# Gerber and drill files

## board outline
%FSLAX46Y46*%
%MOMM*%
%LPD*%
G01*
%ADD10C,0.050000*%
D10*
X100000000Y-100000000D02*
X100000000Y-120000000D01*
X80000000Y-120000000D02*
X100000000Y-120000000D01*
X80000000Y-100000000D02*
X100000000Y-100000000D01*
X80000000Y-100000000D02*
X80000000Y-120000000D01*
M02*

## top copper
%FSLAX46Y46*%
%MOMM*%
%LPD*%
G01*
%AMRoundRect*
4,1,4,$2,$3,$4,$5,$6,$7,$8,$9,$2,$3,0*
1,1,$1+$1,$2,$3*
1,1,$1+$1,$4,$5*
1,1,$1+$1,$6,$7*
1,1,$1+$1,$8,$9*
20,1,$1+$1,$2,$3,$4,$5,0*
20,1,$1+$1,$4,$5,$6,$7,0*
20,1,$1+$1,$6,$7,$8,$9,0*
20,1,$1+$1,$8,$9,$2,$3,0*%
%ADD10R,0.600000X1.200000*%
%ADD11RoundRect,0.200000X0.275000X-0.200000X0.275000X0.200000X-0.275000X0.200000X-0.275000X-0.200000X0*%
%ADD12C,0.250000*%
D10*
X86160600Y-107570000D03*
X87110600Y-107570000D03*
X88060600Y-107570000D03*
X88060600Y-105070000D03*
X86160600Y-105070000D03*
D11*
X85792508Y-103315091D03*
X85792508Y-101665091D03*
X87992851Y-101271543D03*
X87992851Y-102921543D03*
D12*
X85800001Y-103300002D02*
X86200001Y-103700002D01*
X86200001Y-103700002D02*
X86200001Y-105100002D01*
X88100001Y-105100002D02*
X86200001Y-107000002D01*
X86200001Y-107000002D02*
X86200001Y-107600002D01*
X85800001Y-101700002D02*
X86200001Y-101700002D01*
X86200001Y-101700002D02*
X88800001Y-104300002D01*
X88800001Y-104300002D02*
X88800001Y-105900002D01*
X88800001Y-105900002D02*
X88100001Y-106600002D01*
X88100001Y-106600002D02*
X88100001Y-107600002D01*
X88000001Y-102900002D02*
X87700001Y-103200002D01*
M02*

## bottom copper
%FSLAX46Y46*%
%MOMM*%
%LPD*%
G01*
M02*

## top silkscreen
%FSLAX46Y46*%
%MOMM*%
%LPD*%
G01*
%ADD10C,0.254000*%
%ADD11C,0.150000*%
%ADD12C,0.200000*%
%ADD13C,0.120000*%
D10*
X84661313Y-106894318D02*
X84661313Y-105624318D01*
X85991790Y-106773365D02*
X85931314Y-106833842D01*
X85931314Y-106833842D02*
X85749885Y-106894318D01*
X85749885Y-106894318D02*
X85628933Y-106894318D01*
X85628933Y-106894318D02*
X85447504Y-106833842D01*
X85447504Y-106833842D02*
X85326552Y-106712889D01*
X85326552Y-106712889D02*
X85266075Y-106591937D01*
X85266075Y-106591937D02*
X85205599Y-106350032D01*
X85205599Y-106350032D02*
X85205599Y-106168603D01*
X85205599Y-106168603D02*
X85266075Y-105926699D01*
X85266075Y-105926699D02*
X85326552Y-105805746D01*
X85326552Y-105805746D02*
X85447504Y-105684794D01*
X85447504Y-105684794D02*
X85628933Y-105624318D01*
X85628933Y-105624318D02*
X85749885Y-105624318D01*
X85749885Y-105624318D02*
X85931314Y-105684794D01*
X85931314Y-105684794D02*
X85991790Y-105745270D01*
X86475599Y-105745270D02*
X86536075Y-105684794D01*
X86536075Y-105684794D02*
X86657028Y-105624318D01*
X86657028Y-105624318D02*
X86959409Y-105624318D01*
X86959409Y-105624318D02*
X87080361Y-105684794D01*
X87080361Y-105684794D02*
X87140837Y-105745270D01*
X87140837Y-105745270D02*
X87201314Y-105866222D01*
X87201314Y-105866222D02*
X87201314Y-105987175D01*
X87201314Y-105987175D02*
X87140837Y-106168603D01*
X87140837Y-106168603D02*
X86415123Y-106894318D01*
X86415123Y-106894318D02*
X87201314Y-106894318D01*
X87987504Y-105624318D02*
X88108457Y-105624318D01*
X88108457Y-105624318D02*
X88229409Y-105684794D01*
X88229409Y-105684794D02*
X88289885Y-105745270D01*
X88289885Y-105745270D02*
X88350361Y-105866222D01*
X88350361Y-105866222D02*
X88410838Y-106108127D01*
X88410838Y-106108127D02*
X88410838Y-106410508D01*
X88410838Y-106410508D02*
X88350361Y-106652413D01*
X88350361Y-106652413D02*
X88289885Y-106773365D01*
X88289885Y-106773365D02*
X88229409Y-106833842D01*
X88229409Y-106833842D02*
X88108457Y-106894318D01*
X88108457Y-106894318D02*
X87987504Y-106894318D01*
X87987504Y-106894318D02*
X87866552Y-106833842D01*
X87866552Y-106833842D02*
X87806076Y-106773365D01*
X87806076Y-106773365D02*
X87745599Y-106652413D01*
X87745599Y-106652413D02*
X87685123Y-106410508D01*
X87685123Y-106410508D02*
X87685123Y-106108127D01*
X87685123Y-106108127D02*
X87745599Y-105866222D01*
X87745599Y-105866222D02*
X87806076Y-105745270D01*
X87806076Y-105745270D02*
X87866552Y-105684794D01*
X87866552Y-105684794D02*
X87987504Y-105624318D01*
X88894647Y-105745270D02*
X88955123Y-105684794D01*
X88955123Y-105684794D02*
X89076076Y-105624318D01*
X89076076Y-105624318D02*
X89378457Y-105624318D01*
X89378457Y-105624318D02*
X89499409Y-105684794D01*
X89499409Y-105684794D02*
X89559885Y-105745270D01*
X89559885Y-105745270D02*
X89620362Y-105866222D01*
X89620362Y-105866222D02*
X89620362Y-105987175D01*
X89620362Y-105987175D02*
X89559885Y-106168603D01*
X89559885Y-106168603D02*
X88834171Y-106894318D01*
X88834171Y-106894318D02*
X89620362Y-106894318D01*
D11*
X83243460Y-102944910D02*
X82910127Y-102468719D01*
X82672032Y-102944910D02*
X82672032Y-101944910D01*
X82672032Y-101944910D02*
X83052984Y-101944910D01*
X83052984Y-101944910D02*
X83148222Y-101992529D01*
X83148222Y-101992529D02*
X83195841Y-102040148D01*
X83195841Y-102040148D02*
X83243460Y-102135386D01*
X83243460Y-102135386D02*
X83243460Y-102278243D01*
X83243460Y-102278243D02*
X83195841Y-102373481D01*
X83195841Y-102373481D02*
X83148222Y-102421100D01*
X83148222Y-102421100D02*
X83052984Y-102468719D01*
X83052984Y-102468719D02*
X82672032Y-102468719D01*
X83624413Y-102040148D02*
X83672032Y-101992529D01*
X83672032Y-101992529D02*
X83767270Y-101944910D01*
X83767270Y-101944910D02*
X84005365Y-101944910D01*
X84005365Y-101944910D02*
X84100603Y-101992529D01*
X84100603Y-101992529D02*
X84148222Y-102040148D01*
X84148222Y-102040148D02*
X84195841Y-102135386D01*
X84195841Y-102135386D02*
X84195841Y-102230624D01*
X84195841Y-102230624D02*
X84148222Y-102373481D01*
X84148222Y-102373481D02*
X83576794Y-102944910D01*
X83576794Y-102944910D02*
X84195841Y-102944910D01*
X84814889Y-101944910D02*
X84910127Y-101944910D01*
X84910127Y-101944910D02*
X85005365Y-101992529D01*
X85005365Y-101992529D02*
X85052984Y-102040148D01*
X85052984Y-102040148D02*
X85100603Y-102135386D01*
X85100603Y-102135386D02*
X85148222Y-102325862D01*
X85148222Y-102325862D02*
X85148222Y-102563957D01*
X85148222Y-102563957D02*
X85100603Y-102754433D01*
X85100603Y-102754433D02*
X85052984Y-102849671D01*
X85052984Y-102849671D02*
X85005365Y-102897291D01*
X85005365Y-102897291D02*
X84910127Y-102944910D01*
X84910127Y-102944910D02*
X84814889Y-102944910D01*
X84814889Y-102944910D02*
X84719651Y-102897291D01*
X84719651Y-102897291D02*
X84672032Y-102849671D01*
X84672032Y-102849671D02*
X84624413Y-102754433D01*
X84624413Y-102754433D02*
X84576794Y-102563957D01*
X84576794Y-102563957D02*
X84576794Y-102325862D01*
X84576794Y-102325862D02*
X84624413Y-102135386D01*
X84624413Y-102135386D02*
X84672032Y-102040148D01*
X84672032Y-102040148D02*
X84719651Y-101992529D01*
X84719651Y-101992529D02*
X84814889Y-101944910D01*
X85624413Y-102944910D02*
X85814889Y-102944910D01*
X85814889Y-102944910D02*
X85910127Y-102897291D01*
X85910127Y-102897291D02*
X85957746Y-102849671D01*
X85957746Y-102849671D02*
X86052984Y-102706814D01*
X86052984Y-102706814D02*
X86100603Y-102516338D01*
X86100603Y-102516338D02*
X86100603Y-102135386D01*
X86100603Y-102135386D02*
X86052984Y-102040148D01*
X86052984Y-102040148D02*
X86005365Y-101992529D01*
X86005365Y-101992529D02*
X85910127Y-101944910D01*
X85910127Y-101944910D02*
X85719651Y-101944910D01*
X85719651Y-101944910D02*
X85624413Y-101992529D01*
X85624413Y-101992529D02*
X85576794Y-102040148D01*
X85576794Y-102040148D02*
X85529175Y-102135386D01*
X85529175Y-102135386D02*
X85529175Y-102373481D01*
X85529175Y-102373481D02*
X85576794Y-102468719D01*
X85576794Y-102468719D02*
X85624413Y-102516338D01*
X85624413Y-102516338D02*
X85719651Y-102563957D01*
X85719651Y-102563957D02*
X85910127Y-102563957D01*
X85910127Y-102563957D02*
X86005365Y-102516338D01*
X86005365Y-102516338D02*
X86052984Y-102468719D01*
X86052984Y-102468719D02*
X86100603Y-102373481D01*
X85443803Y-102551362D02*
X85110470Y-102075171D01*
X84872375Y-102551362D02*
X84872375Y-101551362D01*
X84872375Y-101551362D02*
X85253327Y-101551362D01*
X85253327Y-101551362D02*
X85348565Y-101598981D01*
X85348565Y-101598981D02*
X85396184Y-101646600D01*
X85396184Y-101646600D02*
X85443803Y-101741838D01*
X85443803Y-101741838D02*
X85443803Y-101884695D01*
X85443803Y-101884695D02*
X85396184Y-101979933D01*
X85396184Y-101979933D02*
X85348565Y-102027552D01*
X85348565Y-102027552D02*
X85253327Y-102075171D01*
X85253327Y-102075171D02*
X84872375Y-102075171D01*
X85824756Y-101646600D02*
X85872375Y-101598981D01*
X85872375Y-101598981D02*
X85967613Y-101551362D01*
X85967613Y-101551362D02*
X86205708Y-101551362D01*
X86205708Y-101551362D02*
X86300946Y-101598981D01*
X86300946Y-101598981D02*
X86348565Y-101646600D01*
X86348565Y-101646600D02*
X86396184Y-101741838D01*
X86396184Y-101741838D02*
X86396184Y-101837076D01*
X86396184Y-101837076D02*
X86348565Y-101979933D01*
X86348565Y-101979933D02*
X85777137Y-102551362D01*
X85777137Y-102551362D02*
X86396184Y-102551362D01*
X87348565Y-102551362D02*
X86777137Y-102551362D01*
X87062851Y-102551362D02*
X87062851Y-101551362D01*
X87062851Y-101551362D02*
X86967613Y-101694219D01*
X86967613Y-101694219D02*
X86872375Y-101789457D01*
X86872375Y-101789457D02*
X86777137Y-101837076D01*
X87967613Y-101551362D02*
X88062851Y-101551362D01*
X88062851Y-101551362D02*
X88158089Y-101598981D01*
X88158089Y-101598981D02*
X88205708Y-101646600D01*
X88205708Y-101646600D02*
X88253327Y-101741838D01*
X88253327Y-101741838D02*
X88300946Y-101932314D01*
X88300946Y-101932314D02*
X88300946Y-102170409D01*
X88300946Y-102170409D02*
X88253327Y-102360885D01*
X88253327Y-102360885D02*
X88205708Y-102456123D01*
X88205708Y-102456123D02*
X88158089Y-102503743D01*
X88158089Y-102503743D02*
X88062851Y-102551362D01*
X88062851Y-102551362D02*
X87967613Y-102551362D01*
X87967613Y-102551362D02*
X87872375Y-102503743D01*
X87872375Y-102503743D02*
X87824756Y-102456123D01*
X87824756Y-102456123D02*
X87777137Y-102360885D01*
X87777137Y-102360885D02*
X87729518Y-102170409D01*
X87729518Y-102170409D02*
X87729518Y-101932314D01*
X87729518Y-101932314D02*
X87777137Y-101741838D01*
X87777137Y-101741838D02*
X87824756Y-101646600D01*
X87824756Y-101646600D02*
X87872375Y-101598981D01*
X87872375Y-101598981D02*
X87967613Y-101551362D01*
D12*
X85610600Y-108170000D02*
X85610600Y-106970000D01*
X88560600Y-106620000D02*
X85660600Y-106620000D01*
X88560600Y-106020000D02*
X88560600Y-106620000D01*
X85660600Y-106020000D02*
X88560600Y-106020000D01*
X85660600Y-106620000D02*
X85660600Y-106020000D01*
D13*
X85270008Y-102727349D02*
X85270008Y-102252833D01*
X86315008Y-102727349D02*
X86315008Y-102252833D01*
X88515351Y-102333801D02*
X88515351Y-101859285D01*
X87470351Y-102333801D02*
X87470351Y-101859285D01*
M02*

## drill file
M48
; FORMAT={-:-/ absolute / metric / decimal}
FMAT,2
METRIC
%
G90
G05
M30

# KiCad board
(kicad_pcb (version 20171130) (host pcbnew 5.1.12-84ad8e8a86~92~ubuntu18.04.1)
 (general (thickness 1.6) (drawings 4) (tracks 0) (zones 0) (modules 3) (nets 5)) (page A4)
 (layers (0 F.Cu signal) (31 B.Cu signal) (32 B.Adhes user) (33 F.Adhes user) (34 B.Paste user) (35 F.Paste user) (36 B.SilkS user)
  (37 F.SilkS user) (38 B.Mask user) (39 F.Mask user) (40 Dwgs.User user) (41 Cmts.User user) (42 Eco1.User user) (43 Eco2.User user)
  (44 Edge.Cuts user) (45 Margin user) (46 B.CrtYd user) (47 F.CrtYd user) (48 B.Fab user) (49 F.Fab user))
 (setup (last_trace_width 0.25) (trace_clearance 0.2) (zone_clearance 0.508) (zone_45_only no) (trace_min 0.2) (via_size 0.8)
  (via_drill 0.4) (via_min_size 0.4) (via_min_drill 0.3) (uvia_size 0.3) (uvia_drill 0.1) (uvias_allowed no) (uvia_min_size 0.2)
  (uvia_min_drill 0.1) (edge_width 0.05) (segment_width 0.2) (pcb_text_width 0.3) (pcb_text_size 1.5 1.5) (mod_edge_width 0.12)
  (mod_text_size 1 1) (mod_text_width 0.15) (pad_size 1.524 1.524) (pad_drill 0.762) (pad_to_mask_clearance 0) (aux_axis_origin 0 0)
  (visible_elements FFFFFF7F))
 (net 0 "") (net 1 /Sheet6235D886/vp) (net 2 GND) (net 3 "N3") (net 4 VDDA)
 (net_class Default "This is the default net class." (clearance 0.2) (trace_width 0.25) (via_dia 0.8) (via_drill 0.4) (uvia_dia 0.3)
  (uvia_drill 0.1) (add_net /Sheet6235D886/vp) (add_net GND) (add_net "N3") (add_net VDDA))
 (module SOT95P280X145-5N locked (layer F.Cu) (at 87.110600 106.320000 90.000000)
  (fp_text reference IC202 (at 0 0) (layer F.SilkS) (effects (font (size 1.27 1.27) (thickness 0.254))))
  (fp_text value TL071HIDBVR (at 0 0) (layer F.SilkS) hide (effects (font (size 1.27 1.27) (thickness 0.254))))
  (fp_line (start -1.85 -1.5) (end -0.65 -1.5) (layer F.SilkS) (width 0.2))
  (fp_line (start -0.3 1.45) (end -0.3 -1.45) (layer F.SilkS) (width 0.2))
  (fp_line (start 0.3 1.45) (end -0.3 1.45) (layer F.SilkS) (width 0.2))
  (fp_line (start 0.3 -1.45) (end 0.3 1.45) (layer F.SilkS) (width 0.2))
  (fp_line (start -0.3 -1.45) (end 0.3 -1.45) (layer F.SilkS) (width 0.2))
  (pad 1 smd rect (at -1.25 -0.95 180.000000) (size 0.6 1.2) (layers F.Cu F.Mask F.Paste) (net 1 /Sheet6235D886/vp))
  (pad 2 smd rect (at -1.25 0 180.000000) (size 0.6 1.2) (layers F.Cu F.Mask F.Paste) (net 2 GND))
  (pad 3 smd rect (at -1.25 0.95 180.000000) (size 0.6 1.2) (layers F.Cu F.Mask F.Paste) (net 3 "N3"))
  (pad 4 smd rect (at 1.25 0.95 180.000000) (size 0.6 1.2) (layers F.Cu F.Mask F.Paste) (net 1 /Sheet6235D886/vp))
  (pad 5 smd rect (at 1.25 -0.95 180.000000) (size 0.6 1.2) (layers F.Cu F.Mask F.Paste) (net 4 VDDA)))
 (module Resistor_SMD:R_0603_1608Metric (layer F.Cu) (at 85.792508 102.490091 90.000000)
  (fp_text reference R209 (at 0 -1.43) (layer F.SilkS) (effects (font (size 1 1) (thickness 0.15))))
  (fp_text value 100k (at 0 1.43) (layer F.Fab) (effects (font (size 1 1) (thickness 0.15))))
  (fp_line (start -0.237258 -0.5225) (end 0.237258 -0.5225) (layer F.SilkS) (width 0.12))
  (fp_line (start -0.237258 0.5225) (end 0.237258 0.5225) (layer F.SilkS) (width 0.12))
  (pad 1 smd roundrect (at -0.825 0 90.000000) (size 0.8 0.95) (layers F.Cu F.Mask F.Paste) (roundrect_rratio 0.25) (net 4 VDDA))
  (pad 2 smd roundrect (at 0.825 0 90.000000) (size 0.8 0.95) (layers F.Cu F.Mask F.Paste) (roundrect_rratio 0.25) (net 3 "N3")))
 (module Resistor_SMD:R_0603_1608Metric (layer F.Cu) (at 87.992851 102.096543 90.000000)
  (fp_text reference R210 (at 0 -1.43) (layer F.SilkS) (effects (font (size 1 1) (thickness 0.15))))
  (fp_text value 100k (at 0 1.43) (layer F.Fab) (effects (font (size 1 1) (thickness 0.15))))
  (fp_line (start -0.237258 0.5225) (end 0.237258 0.5225) (layer F.SilkS) (width 0.12))
  (fp_line (start -0.237258 -0.5225) (end 0.237258 -0.5225) (layer F.SilkS) (width 0.12))
  (pad 2 smd roundrect (at 0.825 0 90.000000) (size 0.8 0.95) (layers F.Cu F.Mask F.Paste) (roundrect_rratio 0.25) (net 2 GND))
  (pad 1 smd roundrect (at -0.825 0 90.000000) (size 0.8 0.95) (layers F.Cu F.Mask F.Paste) (roundrect_rratio 0.25) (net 3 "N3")))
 (gr_line (start 100 100) (end 100 120) (layer Edge.Cuts) (width 0.05))
 (gr_line (start 80 120) (end 100 120) (layer Edge.Cuts) (width 0.05))
 (gr_line (start 80 100) (end 100 100) (layer Edge.Cuts) (width 0.05))
 (gr_line (start 80 100) (end 80 120) (layer Edge.Cuts) (width 0.05))
 (segment (start 85.800001 103.300002) (end 86.200001 103.700002) (width 0.250000) (layer F.Cu) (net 4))
 (segment (start 86.200001 103.700002) (end 86.200001 105.100002) (width 0.250000) (layer F.Cu) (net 4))
 (segment (start 88.100001 105.100002) (end 86.200001 107.000002) (width 0.250000) (layer F.Cu) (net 1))
 (segment (start 86.200001 107.000002) (end 86.200001 107.600002) (width 0.250000) (layer F.Cu) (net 1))
 (segment (start 85.800001 101.700002) (end 86.200001 101.700002) (width 0.250000) (layer F.Cu) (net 3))
 (segment (start 86.200001 101.700002) (end 88.800001 104.300002) (width 0.250000) (layer F.Cu) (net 3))
 (segment (start 88.800001 104.300002) (end 88.800001 105.900002) (width 0.250000) (layer F.Cu) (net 3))
 (segment (start 88.800001 105.900002) (end 88.100001 106.600002) (width 0.250000) (layer F.Cu) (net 3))
 (segment (start 88.100001 106.600002) (end 88.100001 107.600002) (width 0.250000) (layer F.Cu) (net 3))
 (segment (start 88.000001 102.900002) (end 87.700001 103.200002) (width 0.250000) (layer F.Cu) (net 3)))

